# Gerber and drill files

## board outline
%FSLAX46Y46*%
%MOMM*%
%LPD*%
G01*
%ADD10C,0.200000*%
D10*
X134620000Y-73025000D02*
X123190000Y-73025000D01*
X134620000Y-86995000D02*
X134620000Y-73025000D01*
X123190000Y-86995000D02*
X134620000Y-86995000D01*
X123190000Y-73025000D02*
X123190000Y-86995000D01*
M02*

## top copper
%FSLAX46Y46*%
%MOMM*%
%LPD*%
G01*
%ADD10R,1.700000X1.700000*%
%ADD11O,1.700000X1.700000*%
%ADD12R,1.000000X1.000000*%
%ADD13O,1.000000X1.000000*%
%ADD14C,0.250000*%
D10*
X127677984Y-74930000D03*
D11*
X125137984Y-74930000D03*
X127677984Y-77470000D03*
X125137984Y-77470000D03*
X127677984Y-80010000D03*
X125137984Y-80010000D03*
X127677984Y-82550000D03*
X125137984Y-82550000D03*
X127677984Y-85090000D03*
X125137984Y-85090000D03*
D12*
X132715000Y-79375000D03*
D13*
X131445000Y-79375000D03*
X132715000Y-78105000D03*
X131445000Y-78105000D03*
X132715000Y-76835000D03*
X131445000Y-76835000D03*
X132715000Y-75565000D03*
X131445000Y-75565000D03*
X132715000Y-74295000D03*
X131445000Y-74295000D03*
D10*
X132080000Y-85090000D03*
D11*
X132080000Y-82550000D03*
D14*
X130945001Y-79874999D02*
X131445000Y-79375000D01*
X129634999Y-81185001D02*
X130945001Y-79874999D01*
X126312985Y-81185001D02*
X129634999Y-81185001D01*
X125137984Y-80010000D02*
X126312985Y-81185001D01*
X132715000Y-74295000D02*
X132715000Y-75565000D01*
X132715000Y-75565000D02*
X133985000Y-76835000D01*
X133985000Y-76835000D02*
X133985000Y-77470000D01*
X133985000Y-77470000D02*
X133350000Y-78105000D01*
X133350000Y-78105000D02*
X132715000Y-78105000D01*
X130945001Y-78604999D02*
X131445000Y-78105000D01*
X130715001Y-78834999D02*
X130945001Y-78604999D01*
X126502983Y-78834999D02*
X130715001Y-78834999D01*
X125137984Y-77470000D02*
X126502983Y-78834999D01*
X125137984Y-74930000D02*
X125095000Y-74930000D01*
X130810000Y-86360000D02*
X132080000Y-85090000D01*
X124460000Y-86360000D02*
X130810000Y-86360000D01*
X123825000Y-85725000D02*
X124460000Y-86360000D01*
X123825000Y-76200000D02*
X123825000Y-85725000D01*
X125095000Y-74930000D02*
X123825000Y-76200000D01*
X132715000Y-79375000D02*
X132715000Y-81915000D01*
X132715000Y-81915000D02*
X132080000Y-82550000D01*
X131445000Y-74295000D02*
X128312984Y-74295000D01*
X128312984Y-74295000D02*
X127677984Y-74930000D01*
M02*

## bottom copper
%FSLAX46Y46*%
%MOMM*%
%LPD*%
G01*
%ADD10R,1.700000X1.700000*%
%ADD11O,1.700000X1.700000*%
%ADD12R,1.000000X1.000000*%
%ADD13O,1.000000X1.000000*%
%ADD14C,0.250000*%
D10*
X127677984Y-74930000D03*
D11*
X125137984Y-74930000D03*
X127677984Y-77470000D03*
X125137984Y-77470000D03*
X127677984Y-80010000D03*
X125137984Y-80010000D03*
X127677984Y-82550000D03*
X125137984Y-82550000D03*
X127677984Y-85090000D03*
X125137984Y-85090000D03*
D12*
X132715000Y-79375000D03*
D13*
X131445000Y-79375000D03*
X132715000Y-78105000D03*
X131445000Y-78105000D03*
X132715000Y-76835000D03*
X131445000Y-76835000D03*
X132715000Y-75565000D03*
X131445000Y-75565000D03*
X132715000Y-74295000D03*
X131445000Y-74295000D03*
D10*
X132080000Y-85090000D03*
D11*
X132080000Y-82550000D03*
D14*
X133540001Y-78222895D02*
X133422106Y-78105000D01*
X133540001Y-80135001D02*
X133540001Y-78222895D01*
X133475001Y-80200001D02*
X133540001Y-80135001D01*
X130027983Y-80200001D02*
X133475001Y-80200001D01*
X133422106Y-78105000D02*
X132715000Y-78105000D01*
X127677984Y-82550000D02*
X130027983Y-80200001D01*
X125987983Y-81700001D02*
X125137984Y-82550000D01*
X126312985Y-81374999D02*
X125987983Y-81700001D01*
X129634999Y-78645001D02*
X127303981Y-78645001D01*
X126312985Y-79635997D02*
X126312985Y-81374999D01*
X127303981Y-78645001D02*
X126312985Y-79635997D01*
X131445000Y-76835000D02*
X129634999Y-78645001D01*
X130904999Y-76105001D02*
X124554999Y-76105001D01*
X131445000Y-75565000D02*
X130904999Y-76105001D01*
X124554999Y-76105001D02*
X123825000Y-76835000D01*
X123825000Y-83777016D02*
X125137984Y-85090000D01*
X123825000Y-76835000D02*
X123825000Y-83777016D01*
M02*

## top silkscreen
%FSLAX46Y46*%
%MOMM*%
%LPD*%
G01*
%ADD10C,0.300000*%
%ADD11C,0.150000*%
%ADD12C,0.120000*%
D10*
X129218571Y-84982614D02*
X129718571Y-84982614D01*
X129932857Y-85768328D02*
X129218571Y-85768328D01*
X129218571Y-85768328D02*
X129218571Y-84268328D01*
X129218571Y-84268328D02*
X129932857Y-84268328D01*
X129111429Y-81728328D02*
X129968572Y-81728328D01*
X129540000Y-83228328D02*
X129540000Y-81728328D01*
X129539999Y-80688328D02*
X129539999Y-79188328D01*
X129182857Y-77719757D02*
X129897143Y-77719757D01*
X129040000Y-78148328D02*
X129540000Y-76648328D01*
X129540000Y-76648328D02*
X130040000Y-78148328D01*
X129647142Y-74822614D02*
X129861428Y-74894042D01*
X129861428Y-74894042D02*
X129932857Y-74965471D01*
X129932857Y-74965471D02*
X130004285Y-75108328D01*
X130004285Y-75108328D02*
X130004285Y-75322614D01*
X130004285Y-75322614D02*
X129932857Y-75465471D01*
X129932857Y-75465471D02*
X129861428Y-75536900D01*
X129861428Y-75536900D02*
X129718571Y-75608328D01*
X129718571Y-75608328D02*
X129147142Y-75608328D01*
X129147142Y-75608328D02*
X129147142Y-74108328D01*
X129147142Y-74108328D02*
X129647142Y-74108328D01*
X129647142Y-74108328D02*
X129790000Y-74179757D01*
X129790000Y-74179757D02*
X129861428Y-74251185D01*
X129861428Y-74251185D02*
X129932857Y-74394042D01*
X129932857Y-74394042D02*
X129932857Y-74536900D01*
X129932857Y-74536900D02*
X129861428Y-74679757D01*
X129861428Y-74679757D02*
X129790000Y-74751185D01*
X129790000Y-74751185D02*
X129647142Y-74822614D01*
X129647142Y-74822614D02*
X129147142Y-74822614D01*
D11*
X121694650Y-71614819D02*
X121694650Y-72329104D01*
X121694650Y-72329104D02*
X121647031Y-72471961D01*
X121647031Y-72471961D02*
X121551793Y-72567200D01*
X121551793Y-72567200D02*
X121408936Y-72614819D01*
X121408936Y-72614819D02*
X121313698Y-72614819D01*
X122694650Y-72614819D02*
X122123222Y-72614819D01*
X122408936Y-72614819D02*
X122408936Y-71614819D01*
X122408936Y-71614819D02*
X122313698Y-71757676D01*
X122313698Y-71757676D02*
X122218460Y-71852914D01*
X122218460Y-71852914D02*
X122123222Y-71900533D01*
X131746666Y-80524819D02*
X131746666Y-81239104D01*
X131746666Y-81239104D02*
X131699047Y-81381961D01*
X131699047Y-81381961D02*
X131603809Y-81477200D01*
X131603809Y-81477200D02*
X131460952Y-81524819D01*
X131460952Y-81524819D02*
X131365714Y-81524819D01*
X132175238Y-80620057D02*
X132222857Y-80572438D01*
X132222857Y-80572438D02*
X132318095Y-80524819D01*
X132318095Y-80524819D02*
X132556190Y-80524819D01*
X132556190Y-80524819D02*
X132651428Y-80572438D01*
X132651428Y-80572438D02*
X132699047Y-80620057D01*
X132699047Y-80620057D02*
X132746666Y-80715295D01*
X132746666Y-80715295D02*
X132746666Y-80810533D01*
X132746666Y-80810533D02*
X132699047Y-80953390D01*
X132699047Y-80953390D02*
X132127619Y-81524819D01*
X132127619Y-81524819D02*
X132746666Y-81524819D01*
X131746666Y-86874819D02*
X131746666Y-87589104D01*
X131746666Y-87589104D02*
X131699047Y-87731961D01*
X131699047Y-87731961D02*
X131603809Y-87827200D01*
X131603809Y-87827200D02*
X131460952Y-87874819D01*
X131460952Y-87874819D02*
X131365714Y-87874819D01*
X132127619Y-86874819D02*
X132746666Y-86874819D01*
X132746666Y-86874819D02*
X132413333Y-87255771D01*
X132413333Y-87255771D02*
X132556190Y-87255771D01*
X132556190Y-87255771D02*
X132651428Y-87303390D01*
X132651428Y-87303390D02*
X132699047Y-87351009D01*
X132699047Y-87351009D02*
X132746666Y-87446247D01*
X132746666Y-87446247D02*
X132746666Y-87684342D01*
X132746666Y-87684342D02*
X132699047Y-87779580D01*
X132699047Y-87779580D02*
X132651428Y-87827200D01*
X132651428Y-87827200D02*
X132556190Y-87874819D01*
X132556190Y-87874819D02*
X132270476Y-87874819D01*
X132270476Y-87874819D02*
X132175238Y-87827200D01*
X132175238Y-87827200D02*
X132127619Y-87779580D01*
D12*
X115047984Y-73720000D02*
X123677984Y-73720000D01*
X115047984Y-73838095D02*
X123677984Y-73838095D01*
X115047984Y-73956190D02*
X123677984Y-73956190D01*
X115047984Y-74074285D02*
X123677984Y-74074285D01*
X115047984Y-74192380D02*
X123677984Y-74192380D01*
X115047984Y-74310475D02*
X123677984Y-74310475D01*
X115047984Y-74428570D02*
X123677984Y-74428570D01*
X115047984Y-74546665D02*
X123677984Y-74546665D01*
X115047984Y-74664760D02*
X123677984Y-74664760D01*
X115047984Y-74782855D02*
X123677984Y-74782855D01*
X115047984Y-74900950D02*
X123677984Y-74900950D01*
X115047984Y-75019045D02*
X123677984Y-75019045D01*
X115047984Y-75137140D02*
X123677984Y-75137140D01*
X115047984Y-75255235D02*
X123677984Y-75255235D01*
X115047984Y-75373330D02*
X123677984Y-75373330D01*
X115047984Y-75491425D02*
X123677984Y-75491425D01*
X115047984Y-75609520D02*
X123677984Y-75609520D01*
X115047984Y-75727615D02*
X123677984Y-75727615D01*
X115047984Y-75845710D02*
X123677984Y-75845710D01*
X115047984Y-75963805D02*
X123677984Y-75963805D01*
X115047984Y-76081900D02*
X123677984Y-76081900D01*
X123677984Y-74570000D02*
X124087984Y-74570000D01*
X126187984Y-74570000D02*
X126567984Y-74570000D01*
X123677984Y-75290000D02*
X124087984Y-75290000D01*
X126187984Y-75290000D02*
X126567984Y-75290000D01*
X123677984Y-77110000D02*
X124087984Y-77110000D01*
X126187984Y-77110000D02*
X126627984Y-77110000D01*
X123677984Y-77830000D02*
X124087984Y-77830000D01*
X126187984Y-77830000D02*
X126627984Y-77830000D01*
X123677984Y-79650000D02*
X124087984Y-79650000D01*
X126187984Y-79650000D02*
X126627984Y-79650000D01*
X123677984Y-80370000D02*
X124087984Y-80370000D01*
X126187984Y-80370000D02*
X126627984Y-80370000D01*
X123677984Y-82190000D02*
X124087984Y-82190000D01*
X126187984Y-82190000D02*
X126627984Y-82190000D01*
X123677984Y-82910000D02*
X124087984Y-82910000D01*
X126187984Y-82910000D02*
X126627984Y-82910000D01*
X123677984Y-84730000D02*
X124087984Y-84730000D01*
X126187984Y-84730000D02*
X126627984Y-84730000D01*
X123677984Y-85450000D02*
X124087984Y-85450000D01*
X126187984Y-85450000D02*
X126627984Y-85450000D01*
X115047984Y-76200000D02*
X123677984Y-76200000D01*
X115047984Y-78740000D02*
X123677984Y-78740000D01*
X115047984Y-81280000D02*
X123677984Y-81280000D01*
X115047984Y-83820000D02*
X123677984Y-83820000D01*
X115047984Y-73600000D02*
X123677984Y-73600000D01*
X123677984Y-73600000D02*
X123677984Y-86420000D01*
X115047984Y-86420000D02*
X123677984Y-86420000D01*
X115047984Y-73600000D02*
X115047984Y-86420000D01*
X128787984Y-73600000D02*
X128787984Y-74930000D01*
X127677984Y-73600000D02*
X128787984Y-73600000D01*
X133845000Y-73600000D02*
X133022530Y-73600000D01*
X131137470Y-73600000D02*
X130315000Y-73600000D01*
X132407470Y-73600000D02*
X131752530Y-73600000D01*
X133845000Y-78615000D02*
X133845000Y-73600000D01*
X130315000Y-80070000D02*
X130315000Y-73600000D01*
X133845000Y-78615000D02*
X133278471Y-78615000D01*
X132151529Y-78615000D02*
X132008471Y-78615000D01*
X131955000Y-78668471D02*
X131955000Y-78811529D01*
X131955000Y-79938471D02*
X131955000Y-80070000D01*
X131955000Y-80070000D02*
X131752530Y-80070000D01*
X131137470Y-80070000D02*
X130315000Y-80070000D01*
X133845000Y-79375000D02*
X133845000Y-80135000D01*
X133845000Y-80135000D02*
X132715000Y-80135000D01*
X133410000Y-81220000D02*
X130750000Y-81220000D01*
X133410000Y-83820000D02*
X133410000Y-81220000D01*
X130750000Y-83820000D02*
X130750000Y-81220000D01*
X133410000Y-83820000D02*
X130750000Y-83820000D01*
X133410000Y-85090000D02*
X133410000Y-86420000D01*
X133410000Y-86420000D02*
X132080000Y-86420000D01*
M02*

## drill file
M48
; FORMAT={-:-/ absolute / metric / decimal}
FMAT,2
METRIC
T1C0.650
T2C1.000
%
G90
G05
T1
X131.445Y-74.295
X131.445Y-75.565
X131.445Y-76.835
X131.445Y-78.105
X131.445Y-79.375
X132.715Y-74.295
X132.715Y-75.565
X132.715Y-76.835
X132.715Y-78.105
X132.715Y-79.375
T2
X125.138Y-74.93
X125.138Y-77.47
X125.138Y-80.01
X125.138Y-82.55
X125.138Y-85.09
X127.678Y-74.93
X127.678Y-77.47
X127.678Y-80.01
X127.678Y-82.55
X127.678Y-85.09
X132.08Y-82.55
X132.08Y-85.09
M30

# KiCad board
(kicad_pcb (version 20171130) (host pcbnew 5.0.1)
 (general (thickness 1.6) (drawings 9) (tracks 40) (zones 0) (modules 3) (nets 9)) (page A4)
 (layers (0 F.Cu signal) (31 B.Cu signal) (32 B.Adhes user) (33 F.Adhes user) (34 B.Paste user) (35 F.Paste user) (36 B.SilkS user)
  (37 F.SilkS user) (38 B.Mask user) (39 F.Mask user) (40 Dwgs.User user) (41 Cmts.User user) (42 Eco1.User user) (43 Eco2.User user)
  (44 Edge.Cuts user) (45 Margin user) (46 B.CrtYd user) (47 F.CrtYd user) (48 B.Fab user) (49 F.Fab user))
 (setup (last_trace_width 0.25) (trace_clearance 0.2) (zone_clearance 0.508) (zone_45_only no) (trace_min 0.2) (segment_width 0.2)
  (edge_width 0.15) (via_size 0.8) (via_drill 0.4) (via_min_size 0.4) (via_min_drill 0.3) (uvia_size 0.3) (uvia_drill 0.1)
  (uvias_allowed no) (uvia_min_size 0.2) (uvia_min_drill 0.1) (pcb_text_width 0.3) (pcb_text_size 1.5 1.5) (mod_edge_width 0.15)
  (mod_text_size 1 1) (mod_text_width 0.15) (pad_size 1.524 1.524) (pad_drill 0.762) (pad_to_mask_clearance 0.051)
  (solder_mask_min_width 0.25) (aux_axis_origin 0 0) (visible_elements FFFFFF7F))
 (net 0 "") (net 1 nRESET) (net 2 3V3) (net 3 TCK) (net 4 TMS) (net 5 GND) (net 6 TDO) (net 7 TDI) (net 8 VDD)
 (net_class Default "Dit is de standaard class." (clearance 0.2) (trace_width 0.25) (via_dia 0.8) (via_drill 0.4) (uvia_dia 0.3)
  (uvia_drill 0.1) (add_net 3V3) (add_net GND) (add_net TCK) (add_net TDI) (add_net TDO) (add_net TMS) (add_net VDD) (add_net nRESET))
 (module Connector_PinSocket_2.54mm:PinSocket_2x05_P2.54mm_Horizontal (layer F.Cu) (at 127.677984 74.93)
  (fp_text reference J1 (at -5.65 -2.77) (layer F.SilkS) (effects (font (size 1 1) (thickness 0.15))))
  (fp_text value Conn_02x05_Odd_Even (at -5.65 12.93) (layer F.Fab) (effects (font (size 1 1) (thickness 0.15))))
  (fp_line (start -12.63 -1.21) (end -4 -1.21) (layer F.SilkS) (width 0.12))
  (fp_line (start -12.63 -1.091905) (end -4 -1.091905) (layer F.SilkS) (width 0.12))
  (fp_line (start -12.63 -0.97381) (end -4 -0.97381) (layer F.SilkS) (width 0.12))
  (fp_line (start -12.63 -0.855715) (end -4 -0.855715) (layer F.SilkS) (width 0.12))
  (fp_line (start -12.63 -0.73762) (end -4 -0.73762) (layer F.SilkS) (width 0.12))
  (fp_line (start -12.63 -0.619525) (end -4 -0.619525) (layer F.SilkS) (width 0.12))
  (fp_line (start -12.63 -0.50143) (end -4 -0.50143) (layer F.SilkS) (width 0.12))
  (fp_line (start -12.63 -0.383335) (end -4 -0.383335) (layer F.SilkS) (width 0.12))
  (fp_line (start -12.63 -0.26524) (end -4 -0.26524) (layer F.SilkS) (width 0.12))
  (fp_line (start -12.63 -0.147145) (end -4 -0.147145) (layer F.SilkS) (width 0.12))
  (fp_line (start -12.63 -0.02905) (end -4 -0.02905) (layer F.SilkS) (width 0.12))
  (fp_line (start -12.63 0.089045) (end -4 0.089045) (layer F.SilkS) (width 0.12))
  (fp_line (start -12.63 0.20714) (end -4 0.20714) (layer F.SilkS) (width 0.12))
  (fp_line (start -12.63 0.325235) (end -4 0.325235) (layer F.SilkS) (width 0.12))
  (fp_line (start -12.63 0.44333) (end -4 0.44333) (layer F.SilkS) (width 0.12))
  (fp_line (start -12.63 0.561425) (end -4 0.561425) (layer F.SilkS) (width 0.12))
  (fp_line (start -12.63 0.67952) (end -4 0.67952) (layer F.SilkS) (width 0.12))
  (fp_line (start -12.63 0.797615) (end -4 0.797615) (layer F.SilkS) (width 0.12))
  (fp_line (start -12.63 0.91571) (end -4 0.91571) (layer F.SilkS) (width 0.12))
  (fp_line (start -12.63 1.033805) (end -4 1.033805) (layer F.SilkS) (width 0.12))
  (fp_line (start -12.63 1.1519) (end -4 1.1519) (layer F.SilkS) (width 0.12))
  (fp_line (start -4 -0.36) (end -3.59 -0.36) (layer F.SilkS) (width 0.12))
  (fp_line (start -1.49 -0.36) (end -1.11 -0.36) (layer F.SilkS) (width 0.12))
  (fp_line (start -4 0.36) (end -3.59 0.36) (layer F.SilkS) (width 0.12))
  (fp_line (start -1.49 0.36) (end -1.11 0.36) (layer F.SilkS) (width 0.12))
  (fp_line (start -4 2.18) (end -3.59 2.18) (layer F.SilkS) (width 0.12))
  (fp_line (start -1.49 2.18) (end -1.05 2.18) (layer F.SilkS) (width 0.12))
  (fp_line (start -4 2.9) (end -3.59 2.9) (layer F.SilkS) (width 0.12))
  (fp_line (start -1.49 2.9) (end -1.05 2.9) (layer F.SilkS) (width 0.12))
  (fp_line (start -4 4.72) (end -3.59 4.72) (layer F.SilkS) (width 0.12))
  (fp_line (start -1.49 4.72) (end -1.05 4.72) (layer F.SilkS) (width 0.12))
  (fp_line (start -4 5.44) (end -3.59 5.44) (layer F.SilkS) (width 0.12))
  (fp_line (start -1.49 5.44) (end -1.05 5.44) (layer F.SilkS) (width 0.12))
  (fp_line (start -4 7.26) (end -3.59 7.26) (layer F.SilkS) (width 0.12))
  (fp_line (start -1.49 7.26) (end -1.05 7.26) (layer F.SilkS) (width 0.12))
  (fp_line (start -4 7.98) (end -3.59 7.98) (layer F.SilkS) (width 0.12))
  (fp_line (start -1.49 7.98) (end -1.05 7.98) (layer F.SilkS) (width 0.12))
  (fp_line (start -4 9.8) (end -3.59 9.8) (layer F.SilkS) (width 0.12))
  (fp_line (start -1.49 9.8) (end -1.05 9.8) (layer F.SilkS) (width 0.12))
  (fp_line (start -4 10.52) (end -3.59 10.52) (layer F.SilkS) (width 0.12))
  (fp_line (start -1.49 10.52) (end -1.05 10.52) (layer F.SilkS) (width 0.12))
  (fp_line (start -12.63 1.27) (end -4 1.27) (layer F.SilkS) (width 0.12))
  (fp_line (start -12.63 3.81) (end -4 3.81) (layer F.SilkS) (width 0.12))
  (fp_line (start -12.63 6.35) (end -4 6.35) (layer F.SilkS) (width 0.12))
  (fp_line (start -12.63 8.89) (end -4 8.89) (layer F.SilkS) (width 0.12))
  (fp_line (start -12.63 -1.33) (end -4 -1.33) (layer F.SilkS) (width 0.12))
  (fp_line (start -4 -1.33) (end -4 11.49) (layer F.SilkS) (width 0.12))
  (fp_line (start -12.63 11.49) (end -4 11.49) (layer F.SilkS) (width 0.12))
  (fp_line (start -12.63 -1.33) (end -12.63 11.49) (layer F.SilkS) (width 0.12))
  (fp_line (start 1.11 -1.33) (end 1.11 0) (layer F.SilkS) (width 0.12))
  (fp_line (start 0 -1.33) (end 1.11 -1.33) (layer F.SilkS) (width 0.12))
  (pad 1 thru_hole rect (at 0 0) (size 1.7 1.7) (drill 1) (layers *.Cu *.Mask) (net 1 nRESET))
  (pad 2 thru_hole oval (at -2.54 0) (size 1.7 1.7) (drill 1) (layers *.Cu *.Mask) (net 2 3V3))
  (pad 3 thru_hole oval (at 0 2.54) (size 1.7 1.7) (drill 1) (layers *.Cu *.Mask))
  (pad 4 thru_hole oval (at -2.54 2.54) (size 1.7 1.7) (drill 1) (layers *.Cu *.Mask) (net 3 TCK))
  (pad 5 thru_hole oval (at 0 5.08) (size 1.7 1.7) (drill 1) (layers *.Cu *.Mask))
  (pad 6 thru_hole oval (at -2.54 5.08) (size 1.7 1.7) (drill 1) (layers *.Cu *.Mask) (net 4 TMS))
  (pad 7 thru_hole oval (at 0 7.62) (size 1.7 1.7) (drill 1) (layers *.Cu *.Mask) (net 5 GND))
  (pad 8 thru_hole oval (at -2.54 7.62) (size 1.7 1.7) (drill 1) (layers *.Cu *.Mask) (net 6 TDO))
  (pad 9 thru_hole oval (at 0 10.16) (size 1.7 1.7) (drill 1) (layers *.Cu *.Mask))
  (pad 10 thru_hole oval (at -2.54 10.16) (size 1.7 1.7) (drill 1) (layers *.Cu *.Mask) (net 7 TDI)))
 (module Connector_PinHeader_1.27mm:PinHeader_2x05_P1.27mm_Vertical (layer F.Cu) (at 132.715 79.375 180)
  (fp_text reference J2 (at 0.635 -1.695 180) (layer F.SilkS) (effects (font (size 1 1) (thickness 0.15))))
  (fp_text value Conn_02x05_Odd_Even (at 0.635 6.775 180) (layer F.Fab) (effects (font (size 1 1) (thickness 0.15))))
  (fp_line (start -1.13 5.775) (end -0.30753 5.775) (layer F.SilkS) (width 0.12))
  (fp_line (start 1.57753 5.775) (end 2.4 5.775) (layer F.SilkS) (width 0.12))
  (fp_line (start 0.30753 5.775) (end 0.96247 5.775) (layer F.SilkS) (width 0.12))
  (fp_line (start -1.13 0.76) (end -1.13 5.775) (layer F.SilkS) (width 0.12))
  (fp_line (start 2.4 -0.695) (end 2.4 5.775) (layer F.SilkS) (width 0.12))
  (fp_line (start -1.13 0.76) (end -0.563471 0.76) (layer F.SilkS) (width 0.12))
  (fp_line (start 0.563471 0.76) (end 0.706529 0.76) (layer F.SilkS) (width 0.12))
  (fp_line (start 0.76 0.706529) (end 0.76 0.563471) (layer F.SilkS) (width 0.12))
  (fp_line (start 0.76 -0.563471) (end 0.76 -0.695) (layer F.SilkS) (width 0.12))
  (fp_line (start 0.76 -0.695) (end 0.96247 -0.695) (layer F.SilkS) (width 0.12))
  (fp_line (start 1.57753 -0.695) (end 2.4 -0.695) (layer F.SilkS) (width 0.12))
  (fp_line (start -1.13 0) (end -1.13 -0.76) (layer F.SilkS) (width 0.12))
  (fp_line (start -1.13 -0.76) (end 0 -0.76) (layer F.SilkS) (width 0.12))
  (pad 1 thru_hole rect (at 0 0 180) (size 1 1) (drill 0.65) (layers *.Cu *.Mask) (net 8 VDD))
  (pad 2 thru_hole oval (at 1.27 0 180) (size 1 1) (drill 0.65) (layers *.Cu *.Mask) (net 4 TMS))
  (pad 3 thru_hole oval (at 0 1.27 180) (size 1 1) (drill 0.65) (layers *.Cu *.Mask) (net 5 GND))
  (pad 4 thru_hole oval (at 1.27 1.27 180) (size 1 1) (drill 0.65) (layers *.Cu *.Mask) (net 3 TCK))
  (pad 5 thru_hole oval (at 0 2.54 180) (size 1 1) (drill 0.65) (layers *.Cu *.Mask))
  (pad 6 thru_hole oval (at 1.27 2.54 180) (size 1 1) (drill 0.65) (layers *.Cu *.Mask) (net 6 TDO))
  (pad 7 thru_hole oval (at 0 3.81 180) (size 1 1) (drill 0.65) (layers *.Cu *.Mask) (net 5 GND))
  (pad 8 thru_hole oval (at 1.27 3.81 180) (size 1 1) (drill 0.65) (layers *.Cu *.Mask) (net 7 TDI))
  (pad 9 thru_hole oval (at 0 5.08 180) (size 1 1) (drill 0.65) (layers *.Cu *.Mask) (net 5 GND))
  (pad 10 thru_hole oval (at 1.27 5.08 180) (size 1 1) (drill 0.65) (layers *.Cu *.Mask) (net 1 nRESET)))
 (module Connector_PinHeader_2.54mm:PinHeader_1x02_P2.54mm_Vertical (layer F.Cu) (at 132.08 85.09 180)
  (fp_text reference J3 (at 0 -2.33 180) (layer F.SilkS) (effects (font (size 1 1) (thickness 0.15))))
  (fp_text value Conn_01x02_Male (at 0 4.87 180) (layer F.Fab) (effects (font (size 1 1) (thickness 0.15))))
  (fp_line (start -1.33 3.87) (end 1.33 3.87) (layer F.SilkS) (width 0.12))
  (fp_line (start -1.33 1.27) (end -1.33 3.87) (layer F.SilkS) (width 0.12))
  (fp_line (start 1.33 1.27) (end 1.33 3.87) (layer F.SilkS) (width 0.12))
  (fp_line (start -1.33 1.27) (end 1.33 1.27) (layer F.SilkS) (width 0.12))
  (fp_line (start -1.33 0) (end -1.33 -1.33) (layer F.SilkS) (width 0.12))
  (fp_line (start -1.33 -1.33) (end 0 -1.33) (layer F.SilkS) (width 0.12))
  (pad 1 thru_hole rect (at 0 0 180) (size 1.7 1.7) (drill 1) (layers *.Cu *.Mask) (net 2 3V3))
  (pad 2 thru_hole oval (at 0 2.54 180) (size 1.7 1.7) (drill 1) (layers *.Cu *.Mask) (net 8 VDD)))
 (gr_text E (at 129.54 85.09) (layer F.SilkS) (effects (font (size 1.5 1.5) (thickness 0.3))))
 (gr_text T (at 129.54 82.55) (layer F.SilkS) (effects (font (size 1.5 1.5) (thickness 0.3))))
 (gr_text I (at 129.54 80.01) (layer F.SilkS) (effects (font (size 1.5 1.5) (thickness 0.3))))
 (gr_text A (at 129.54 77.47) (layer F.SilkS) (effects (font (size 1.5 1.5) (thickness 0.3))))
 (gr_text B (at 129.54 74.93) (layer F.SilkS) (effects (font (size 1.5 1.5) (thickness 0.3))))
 (gr_line (start 134.62 73.025) (end 123.19 73.025) (layer Edge.Cuts) (width 0.2))
 (gr_line (start 134.62 86.995) (end 134.62 73.025) (layer Edge.Cuts) (width 0.2))
 (gr_line (start 123.19 86.995) (end 134.62 86.995) (layer Edge.Cuts) (width 0.2))
 (gr_line (start 123.19 73.025) (end 123.19 86.995) (layer Edge.Cuts) (width 0.2))
 (segment (start 130.945001 79.874999) (end 131.445 79.375) (width 0.25) (layer F.Cu) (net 4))
 (segment (start 129.634999 81.185001) (end 130.945001 79.874999) (width 0.25) (layer F.Cu) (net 4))
 (segment (start 126.312985 81.185001) (end 129.634999 81.185001) (width 0.25) (layer F.Cu) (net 4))
 (segment (start 125.137984 80.01) (end 126.312985 81.185001) (width 0.25) (layer F.Cu) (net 4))
 (segment (start 132.715 74.295) (end 132.715 75.565) (width 0.25) (layer F.Cu) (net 5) (status C00000))
 (segment (start 132.715 75.565) (end 133.985 76.835) (width 0.25) (layer F.Cu) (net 5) (status 400000))
 (segment (start 133.985 76.835) (end 133.985 77.47) (width 0.25) (layer F.Cu) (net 5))
 (segment (start 133.985 77.47) (end 133.35 78.105) (width 0.25) (layer F.Cu) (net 5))
 (segment (start 133.35 78.105) (end 132.715 78.105) (width 0.25) (layer F.Cu) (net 5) (status 800000))
 (segment (start 133.540001 78.222895) (end 133.422106 78.105) (width 0.25) (layer B.Cu) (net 5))
 (segment (start 133.540001 80.135001) (end 133.540001 78.222895) (width 0.25) (layer B.Cu) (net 5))
 (segment (start 133.475001 80.200001) (end 133.540001 80.135001) (width 0.25) (layer B.Cu) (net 5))
 (segment (start 130.027983 80.200001) (end 133.475001 80.200001) (width 0.25) (layer B.Cu) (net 5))
 (segment (start 133.422106 78.105) (end 132.715 78.105) (width 0.25) (layer B.Cu) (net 5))
 (segment (start 127.677984 82.55) (end 130.027983 80.200001) (width 0.25) (layer B.Cu) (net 5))
 (segment (start 130.945001 78.604999) (end 131.445 78.105) (width 0.25) (layer F.Cu) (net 3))
 (segment (start 130.715001 78.834999) (end 130.945001 78.604999) (width 0.25) (layer F.Cu) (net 3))
 (segment (start 126.502983 78.834999) (end 130.715001 78.834999) (width 0.25) (layer F.Cu) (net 3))
 (segment (start 125.137984 77.47) (end 126.502983 78.834999) (width 0.25) (layer F.Cu) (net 3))
 (segment (start 125.137984 74.93) (end 125.095 74.93) (width 0.25) (layer F.Cu) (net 2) (status C00000))
 (segment (start 130.81 86.36) (end 132.08 85.09) (width 0.25) (layer F.Cu) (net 2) (status 800000))
 (segment (start 124.46 86.36) (end 130.81 86.36) (width 0.25) (layer F.Cu) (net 2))
 (segment (start 123.825 85.725) (end 124.46 86.36) (width 0.25) (layer F.Cu) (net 2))
 (segment (start 123.825 76.2) (end 123.825 85.725) (width 0.25) (layer F.Cu) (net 2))
 (segment (start 125.095 74.93) (end 123.825 76.2) (width 0.25) (layer F.Cu) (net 2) (status 400000))
 (segment (start 132.715 79.375) (end 132.715 81.915) (width 0.25) (layer F.Cu) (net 8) (status C00000))
 (segment (start 132.715 81.915) (end 132.08 82.55) (width 0.25) (layer F.Cu) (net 8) (status C00000))
 (segment (start 131.445 74.295) (end 128.312984 74.295) (width 0.25) (layer F.Cu) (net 1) (status C00000))
 (segment (start 128.312984 74.295) (end 127.677984 74.93) (width 0.25) (layer F.Cu) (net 1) (status C00000))
 (segment (start 125.987983 81.700001) (end 125.137984 82.55) (width 0.25) (layer B.Cu) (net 6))
 (segment (start 126.312985 81.374999) (end 125.987983 81.700001) (width 0.25) (layer B.Cu) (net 6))
 (segment (start 129.634999 78.645001) (end 127.303981 78.645001) (width 0.25) (layer B.Cu) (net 6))
 (segment (start 126.312985 79.635997) (end 126.312985 81.374999) (width 0.25) (layer B.Cu) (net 6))
 (segment (start 127.303981 78.645001) (end 126.312985 79.635997) (width 0.25) (layer B.Cu) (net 6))
 (segment (start 131.445 76.835) (end 129.634999 78.645001) (width 0.25) (layer B.Cu) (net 6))
 (segment (start 130.904999 76.105001) (end 124.554999 76.105001) (width 0.25) (layer B.Cu) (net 7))
 (segment (start 131.445 75.565) (end 130.904999 76.105001) (width 0.25) (layer B.Cu) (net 7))
 (segment (start 124.554999 76.105001) (end 123.825 76.835) (width 0.25) (layer B.Cu) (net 7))
 (segment (start 123.825 83.777016) (end 125.137984 85.09) (width 0.25) (layer B.Cu) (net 7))
 (segment (start 123.825 76.835) (end 123.825 83.777016) (width 0.25) (layer B.Cu) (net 7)))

